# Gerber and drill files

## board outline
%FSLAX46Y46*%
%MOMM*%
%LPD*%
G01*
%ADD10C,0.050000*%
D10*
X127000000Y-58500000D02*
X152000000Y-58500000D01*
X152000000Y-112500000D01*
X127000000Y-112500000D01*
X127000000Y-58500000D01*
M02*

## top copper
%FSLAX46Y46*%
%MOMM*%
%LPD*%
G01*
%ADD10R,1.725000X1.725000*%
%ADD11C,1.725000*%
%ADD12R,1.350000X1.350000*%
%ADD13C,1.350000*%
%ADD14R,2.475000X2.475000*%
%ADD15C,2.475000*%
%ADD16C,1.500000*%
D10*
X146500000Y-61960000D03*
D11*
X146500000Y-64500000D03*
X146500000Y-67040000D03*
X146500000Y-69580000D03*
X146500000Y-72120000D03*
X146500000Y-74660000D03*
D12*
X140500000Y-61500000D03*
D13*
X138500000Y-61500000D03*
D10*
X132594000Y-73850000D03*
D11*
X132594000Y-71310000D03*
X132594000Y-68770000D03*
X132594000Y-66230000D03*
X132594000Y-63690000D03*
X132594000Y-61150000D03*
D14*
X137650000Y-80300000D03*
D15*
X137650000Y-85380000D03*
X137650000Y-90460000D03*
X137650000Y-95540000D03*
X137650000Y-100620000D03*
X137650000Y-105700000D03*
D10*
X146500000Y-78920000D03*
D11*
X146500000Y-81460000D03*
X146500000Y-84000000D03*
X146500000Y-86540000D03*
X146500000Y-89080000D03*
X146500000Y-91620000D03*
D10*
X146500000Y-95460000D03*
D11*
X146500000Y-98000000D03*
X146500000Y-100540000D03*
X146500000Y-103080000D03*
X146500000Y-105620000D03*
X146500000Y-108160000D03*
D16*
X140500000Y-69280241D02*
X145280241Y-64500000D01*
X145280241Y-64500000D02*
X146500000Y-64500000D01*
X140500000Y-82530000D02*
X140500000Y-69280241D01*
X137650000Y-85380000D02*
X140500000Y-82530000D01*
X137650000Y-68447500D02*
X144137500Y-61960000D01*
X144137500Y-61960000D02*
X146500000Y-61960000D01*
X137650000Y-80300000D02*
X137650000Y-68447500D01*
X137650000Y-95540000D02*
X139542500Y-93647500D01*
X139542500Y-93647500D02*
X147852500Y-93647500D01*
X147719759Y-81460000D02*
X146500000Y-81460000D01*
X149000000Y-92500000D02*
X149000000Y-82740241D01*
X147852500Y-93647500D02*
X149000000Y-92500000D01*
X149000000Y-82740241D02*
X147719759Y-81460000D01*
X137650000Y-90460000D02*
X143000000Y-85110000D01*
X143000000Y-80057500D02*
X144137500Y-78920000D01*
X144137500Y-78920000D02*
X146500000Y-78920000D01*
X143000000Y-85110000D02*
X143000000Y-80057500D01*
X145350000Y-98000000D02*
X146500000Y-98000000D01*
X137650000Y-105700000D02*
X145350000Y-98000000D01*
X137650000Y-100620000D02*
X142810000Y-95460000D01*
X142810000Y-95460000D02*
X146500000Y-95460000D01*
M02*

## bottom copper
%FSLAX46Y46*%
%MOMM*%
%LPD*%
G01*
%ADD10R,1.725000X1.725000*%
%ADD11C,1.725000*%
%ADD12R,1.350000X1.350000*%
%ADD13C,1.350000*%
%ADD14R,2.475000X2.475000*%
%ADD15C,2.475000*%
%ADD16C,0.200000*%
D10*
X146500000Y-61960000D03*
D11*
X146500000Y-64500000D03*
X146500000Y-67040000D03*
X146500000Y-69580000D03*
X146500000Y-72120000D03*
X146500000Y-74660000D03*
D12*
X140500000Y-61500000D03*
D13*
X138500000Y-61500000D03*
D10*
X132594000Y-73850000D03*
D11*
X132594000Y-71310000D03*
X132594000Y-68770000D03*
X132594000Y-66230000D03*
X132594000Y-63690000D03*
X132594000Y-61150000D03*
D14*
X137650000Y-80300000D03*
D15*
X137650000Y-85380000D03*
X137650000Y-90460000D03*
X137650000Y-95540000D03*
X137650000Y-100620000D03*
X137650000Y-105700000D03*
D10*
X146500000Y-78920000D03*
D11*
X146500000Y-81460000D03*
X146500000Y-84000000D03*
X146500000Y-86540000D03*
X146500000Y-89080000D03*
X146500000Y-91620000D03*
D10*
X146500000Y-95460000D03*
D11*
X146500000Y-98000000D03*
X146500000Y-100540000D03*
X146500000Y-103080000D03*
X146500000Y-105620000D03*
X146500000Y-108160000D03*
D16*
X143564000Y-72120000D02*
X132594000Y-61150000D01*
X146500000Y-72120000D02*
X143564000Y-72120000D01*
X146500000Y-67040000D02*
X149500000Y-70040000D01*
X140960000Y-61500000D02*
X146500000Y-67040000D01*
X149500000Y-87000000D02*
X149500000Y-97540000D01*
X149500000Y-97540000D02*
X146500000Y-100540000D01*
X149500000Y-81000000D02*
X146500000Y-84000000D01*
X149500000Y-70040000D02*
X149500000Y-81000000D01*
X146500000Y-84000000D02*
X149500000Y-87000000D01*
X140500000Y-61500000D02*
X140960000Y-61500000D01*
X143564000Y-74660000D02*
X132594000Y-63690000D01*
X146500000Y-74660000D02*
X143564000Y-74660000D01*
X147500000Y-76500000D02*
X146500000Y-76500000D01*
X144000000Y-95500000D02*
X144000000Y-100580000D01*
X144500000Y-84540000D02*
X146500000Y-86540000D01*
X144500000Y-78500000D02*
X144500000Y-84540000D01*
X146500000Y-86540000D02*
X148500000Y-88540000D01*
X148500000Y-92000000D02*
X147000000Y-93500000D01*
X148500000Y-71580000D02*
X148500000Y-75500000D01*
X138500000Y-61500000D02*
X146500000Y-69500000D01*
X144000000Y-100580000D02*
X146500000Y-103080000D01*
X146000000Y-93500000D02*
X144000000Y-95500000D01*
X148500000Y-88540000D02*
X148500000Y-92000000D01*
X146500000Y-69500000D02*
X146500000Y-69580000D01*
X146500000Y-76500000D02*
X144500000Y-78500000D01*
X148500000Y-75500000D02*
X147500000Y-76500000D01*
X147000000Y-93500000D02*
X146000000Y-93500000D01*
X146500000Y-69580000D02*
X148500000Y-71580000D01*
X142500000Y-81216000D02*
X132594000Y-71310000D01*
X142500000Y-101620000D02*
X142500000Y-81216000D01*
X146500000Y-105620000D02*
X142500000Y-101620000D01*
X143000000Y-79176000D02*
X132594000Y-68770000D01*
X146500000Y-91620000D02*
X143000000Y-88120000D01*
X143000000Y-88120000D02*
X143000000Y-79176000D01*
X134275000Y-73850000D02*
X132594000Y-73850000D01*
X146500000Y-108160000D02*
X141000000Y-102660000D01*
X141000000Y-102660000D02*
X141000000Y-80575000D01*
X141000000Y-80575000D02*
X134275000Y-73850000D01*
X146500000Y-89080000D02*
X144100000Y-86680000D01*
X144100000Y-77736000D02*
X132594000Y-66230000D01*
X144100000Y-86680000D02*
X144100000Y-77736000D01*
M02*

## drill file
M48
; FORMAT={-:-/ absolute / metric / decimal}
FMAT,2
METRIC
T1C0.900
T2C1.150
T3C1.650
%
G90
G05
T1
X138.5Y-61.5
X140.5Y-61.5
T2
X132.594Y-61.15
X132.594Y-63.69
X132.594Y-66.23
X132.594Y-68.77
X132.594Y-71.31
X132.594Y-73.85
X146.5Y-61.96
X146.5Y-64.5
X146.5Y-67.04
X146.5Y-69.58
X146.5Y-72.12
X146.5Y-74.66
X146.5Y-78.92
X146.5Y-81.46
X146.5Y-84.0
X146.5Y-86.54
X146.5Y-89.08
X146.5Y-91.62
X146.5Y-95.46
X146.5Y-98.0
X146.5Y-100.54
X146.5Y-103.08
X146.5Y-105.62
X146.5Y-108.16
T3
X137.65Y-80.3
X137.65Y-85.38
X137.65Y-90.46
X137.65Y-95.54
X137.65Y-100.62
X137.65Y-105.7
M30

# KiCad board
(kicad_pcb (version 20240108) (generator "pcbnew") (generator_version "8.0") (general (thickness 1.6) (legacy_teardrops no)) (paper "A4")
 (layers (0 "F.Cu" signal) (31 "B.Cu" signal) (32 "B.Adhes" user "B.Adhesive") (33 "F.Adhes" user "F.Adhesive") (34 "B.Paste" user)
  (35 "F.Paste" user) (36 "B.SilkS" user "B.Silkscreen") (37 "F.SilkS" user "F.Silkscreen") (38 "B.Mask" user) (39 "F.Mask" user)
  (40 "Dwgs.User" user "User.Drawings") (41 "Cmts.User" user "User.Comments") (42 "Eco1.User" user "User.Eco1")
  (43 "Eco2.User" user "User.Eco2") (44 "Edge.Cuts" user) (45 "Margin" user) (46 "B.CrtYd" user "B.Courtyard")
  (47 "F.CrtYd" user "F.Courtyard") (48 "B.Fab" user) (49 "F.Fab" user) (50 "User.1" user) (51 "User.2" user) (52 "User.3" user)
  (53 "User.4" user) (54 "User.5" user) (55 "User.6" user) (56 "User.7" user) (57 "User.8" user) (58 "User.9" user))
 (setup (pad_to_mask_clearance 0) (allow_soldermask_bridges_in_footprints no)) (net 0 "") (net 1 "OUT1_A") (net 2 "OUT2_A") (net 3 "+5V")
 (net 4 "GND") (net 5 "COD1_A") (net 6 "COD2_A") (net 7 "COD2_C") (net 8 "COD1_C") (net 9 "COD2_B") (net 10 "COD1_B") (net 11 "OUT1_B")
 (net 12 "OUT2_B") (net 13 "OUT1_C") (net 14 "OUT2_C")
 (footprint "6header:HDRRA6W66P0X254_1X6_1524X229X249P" (layer "F.Cu") (at 146.5 61.96 -90)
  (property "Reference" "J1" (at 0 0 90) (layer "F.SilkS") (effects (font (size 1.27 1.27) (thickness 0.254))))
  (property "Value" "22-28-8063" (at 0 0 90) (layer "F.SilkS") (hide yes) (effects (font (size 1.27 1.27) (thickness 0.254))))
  (pad "1" thru_hole rect (at 0 0 270) (size 1.725 1.725) (drill 1.15) (layers "*.Cu" "*.Mask") (remove_unused_layers no) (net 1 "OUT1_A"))
  (pad "2" thru_hole circle (at 2.54 0 270) (size 1.725 1.725) (drill 1.15) (layers "*.Cu" "*.Mask") (remove_unused_layers no)
   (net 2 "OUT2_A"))
  (pad "3" thru_hole circle (at 5.08 0 270) (size 1.725 1.725) (drill 1.15) (layers "*.Cu" "*.Mask") (remove_unused_layers no) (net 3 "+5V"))
  (pad "4" thru_hole circle (at 7.62 0 270) (size 1.725 1.725) (drill 1.15) (layers "*.Cu" "*.Mask") (remove_unused_layers no) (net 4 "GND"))
  (pad "5" thru_hole circle (at 10.16 0 270) (size 1.725 1.725) (drill 1.15) (layers "*.Cu" "*.Mask") (remove_unused_layers no)
   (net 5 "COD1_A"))
  (pad "6" thru_hole circle (at 12.7 0 270) (size 1.725 1.725) (drill 1.15) (layers "*.Cu" "*.Mask") (remove_unused_layers no)
   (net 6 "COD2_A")))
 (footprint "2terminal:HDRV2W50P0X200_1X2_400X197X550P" (layer "F.Cu") (at 140.5 61.5)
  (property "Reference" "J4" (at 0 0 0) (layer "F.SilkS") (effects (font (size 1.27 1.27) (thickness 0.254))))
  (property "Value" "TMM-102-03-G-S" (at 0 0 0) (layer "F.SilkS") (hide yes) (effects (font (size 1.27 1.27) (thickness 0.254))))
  (pad "1" thru_hole rect (at 0 0) (size 1.35 1.35) (drill 0.9) (layers "*.Cu" "*.Mask") (remove_unused_layers no) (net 3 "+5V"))
  (pad "2" thru_hole circle (at -2 0) (size 1.35 1.35) (drill 0.9) (layers "*.Cu" "*.Mask") (remove_unused_layers no) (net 4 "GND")))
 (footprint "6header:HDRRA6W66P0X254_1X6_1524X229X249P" (layer "F.Cu") (at 132.594 73.85 90)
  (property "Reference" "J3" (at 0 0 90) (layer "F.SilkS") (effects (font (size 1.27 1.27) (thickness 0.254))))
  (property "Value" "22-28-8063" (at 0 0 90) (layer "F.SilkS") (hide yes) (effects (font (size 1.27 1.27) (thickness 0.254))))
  (pad "1" thru_hole rect (at 0 0 90) (size 1.725 1.725) (drill 1.15) (layers "*.Cu" "*.Mask") (remove_unused_layers no) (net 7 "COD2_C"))
  (pad "2" thru_hole circle (at 2.54 0 90) (size 1.725 1.725) (drill 1.15) (layers "*.Cu" "*.Mask") (remove_unused_layers no)
   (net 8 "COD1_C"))
  (pad "3" thru_hole circle (at 5.08 0 90) (size 1.725 1.725) (drill 1.15) (layers "*.Cu" "*.Mask") (remove_unused_layers no)
   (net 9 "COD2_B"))
  (pad "4" thru_hole circle (at 7.62 0 90) (size 1.725 1.725) (drill 1.15) (layers "*.Cu" "*.Mask") (remove_unused_layers no)
   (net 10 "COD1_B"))
  (pad "5" thru_hole circle (at 10.16 0 90) (size 1.725 1.725) (drill 1.15) (layers "*.Cu" "*.Mask") (remove_unused_layers no)
   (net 6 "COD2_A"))
  (pad "6" thru_hole circle (at 12.7 0 90) (size 1.725 1.725) (drill 1.15) (layers "*.Cu" "*.Mask") (remove_unused_layers no)
   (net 5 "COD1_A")))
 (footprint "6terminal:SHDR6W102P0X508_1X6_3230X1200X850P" (layer "F.Cu") (at 137.65 80.3 -90)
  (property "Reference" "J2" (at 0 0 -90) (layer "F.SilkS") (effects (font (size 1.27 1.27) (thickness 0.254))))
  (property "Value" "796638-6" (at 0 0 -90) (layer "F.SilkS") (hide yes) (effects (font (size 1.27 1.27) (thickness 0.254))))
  (pad "1" thru_hole rect (at 0 0 270) (size 2.475 2.475) (drill 1.65) (layers "*.Cu" "*.Mask") (remove_unused_layers no) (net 1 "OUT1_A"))
  (pad "2" thru_hole circle (at 5.08 0 270) (size 2.475 2.475) (drill 1.65) (layers "*.Cu" "*.Mask") (remove_unused_layers no)
   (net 2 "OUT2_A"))
  (pad "3" thru_hole circle (at 10.16 0 270) (size 2.475 2.475) (drill 1.65) (layers "*.Cu" "*.Mask") (remove_unused_layers no)
   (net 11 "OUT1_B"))
  (pad "4" thru_hole circle (at 15.24 0 270) (size 2.475 2.475) (drill 1.65) (layers "*.Cu" "*.Mask") (remove_unused_layers no)
   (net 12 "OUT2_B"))
  (pad "5" thru_hole circle (at 20.32 0 270) (size 2.475 2.475) (drill 1.65) (layers "*.Cu" "*.Mask") (remove_unused_layers no)
   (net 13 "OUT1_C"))
  (pad "6" thru_hole circle (at 25.4 0 270) (size 2.475 2.475) (drill 1.65) (layers "*.Cu" "*.Mask") (remove_unused_layers no)
   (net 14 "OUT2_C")))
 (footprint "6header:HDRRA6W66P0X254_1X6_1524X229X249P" (layer "F.Cu") (at 146.5 78.92 -90)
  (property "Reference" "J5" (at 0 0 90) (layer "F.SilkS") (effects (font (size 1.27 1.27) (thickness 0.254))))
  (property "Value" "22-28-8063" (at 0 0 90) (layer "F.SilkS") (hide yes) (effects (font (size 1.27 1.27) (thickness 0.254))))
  (pad "1" thru_hole rect (at 0 0 270) (size 1.725 1.725) (drill 1.15) (layers "*.Cu" "*.Mask") (remove_unused_layers no) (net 11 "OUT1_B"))
  (pad "2" thru_hole circle (at 2.54 0 270) (size 1.725 1.725) (drill 1.15) (layers "*.Cu" "*.Mask") (remove_unused_layers no)
   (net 12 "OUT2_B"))
  (pad "3" thru_hole circle (at 5.08 0 270) (size 1.725 1.725) (drill 1.15) (layers "*.Cu" "*.Mask") (remove_unused_layers no) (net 3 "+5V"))
  (pad "4" thru_hole circle (at 7.62 0 270) (size 1.725 1.725) (drill 1.15) (layers "*.Cu" "*.Mask") (remove_unused_layers no) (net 4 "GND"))
  (pad "5" thru_hole circle (at 10.16 0 270) (size 1.725 1.725) (drill 1.15) (layers "*.Cu" "*.Mask") (remove_unused_layers no)
   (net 10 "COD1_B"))
  (pad "6" thru_hole circle (at 12.7 0 270) (size 1.725 1.725) (drill 1.15) (layers "*.Cu" "*.Mask") (remove_unused_layers no)
   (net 9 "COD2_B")))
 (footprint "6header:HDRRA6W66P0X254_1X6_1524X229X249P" (layer "F.Cu") (at 146.5 95.46 -90)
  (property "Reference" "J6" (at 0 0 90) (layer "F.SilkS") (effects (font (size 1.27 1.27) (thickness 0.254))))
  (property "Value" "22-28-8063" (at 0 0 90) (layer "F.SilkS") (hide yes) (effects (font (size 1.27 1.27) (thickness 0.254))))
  (pad "1" thru_hole rect (at 0 0 270) (size 1.725 1.725) (drill 1.15) (layers "*.Cu" "*.Mask") (remove_unused_layers no) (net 13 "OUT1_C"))
  (pad "2" thru_hole circle (at 2.54 0 270) (size 1.725 1.725) (drill 1.15) (layers "*.Cu" "*.Mask") (remove_unused_layers no)
   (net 14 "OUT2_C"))
  (pad "3" thru_hole circle (at 5.08 0 270) (size 1.725 1.725) (drill 1.15) (layers "*.Cu" "*.Mask") (remove_unused_layers no) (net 3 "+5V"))
  (pad "4" thru_hole circle (at 7.62 0 270) (size 1.725 1.725) (drill 1.15) (layers "*.Cu" "*.Mask") (remove_unused_layers no) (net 4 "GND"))
  (pad "5" thru_hole circle (at 10.16 0 270) (size 1.725 1.725) (drill 1.15) (layers "*.Cu" "*.Mask") (remove_unused_layers no)
   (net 8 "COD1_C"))
  (pad "6" thru_hole circle (at 12.7 0 270) (size 1.725 1.725) (drill 1.15) (layers "*.Cu" "*.Mask") (remove_unused_layers no)
   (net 7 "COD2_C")))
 (gr_rect (start 127 58.5) (end 152 112.5) (stroke (width 0.05) (type default)) (fill none) (layer "Edge.Cuts"))
 (segment (start 143.564 72.12) (end 132.594 61.15) (width 0.2) (layer "B.Cu") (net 5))
 (segment (start 146.5 72.12) (end 143.564 72.12) (width 0.2) (layer "B.Cu") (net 5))
 (segment (start 140.5 69.280241) (end 145.280241 64.5) (width 1.5) (layer "F.Cu") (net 2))
 (segment (start 145.280241 64.5) (end 146.5 64.5) (width 1.5) (layer "F.Cu") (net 2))
 (segment (start 140.5 82.53) (end 140.5 69.280241) (width 1.5) (layer "F.Cu") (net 2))
 (segment (start 137.65 85.38) (end 140.5 82.53) (width 1.5) (layer "F.Cu") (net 2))
 (segment (start 137.65 68.4475) (end 144.1375 61.96) (width 1.5) (layer "F.Cu") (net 1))
 (segment (start 144.1375 61.96) (end 146.5 61.96) (width 1.5) (layer "F.Cu") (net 1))
 (segment (start 137.65 80.3) (end 137.65 68.4475) (width 1.5) (layer "F.Cu") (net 1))
 (segment (start 146.5 67.04) (end 149.5 70.04) (width 0.2) (layer "B.Cu") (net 3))
 (segment (start 140.96 61.5) (end 146.5 67.04) (width 0.2) (layer "B.Cu") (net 3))
 (segment (start 149.5 87) (end 149.5 97.54) (width 0.2) (layer "B.Cu") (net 3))
 (segment (start 149.5 97.54) (end 146.5 100.54) (width 0.2) (layer "B.Cu") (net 3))
 (segment (start 149.5 81) (end 146.5 84) (width 0.2) (layer "B.Cu") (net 3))
 (segment (start 149.5 70.04) (end 149.5 81) (width 0.2) (layer "B.Cu") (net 3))
 (segment (start 146.5 84) (end 149.5 87) (width 0.2) (layer "B.Cu") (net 3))
 (segment (start 140.5 61.5) (end 140.96 61.5) (width 0.2) (layer "B.Cu") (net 3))
 (segment (start 143.564 74.66) (end 132.594 63.69) (width 0.2) (layer "B.Cu") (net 6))
 (segment (start 146.5 74.66) (end 143.564 74.66) (width 0.2) (layer "B.Cu") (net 6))
 (segment (start 147.5 76.5) (end 146.5 76.5) (width 0.2) (layer "B.Cu") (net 4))
 (segment (start 144 95.5) (end 144 100.58) (width 0.2) (layer "B.Cu") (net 4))
 (segment (start 144.5 84.54) (end 146.5 86.54) (width 0.2) (layer "B.Cu") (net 4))
 (segment (start 144.5 78.5) (end 144.5 84.54) (width 0.2) (layer "B.Cu") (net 4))
 (segment (start 146.5 86.54) (end 148.5 88.54) (width 0.2) (layer "B.Cu") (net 4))
 (segment (start 148.5 92) (end 147 93.5) (width 0.2) (layer "B.Cu") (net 4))
 (segment (start 148.5 71.58) (end 148.5 75.5) (width 0.2) (layer "B.Cu") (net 4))
 (segment (start 138.5 61.5) (end 146.5 69.5) (width 0.2) (layer "B.Cu") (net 4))
 (segment (start 144 100.58) (end 146.5 103.08) (width 0.2) (layer "B.Cu") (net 4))
 (segment (start 146 93.5) (end 144 95.5) (width 0.2) (layer "B.Cu") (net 4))
 (segment (start 148.5 88.54) (end 148.5 92) (width 0.2) (layer "B.Cu") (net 4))
 (segment (start 146.5 69.5) (end 146.5 69.58) (width 0.2) (layer "B.Cu") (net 4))
 (segment (start 146.5 76.5) (end 144.5 78.5) (width 0.2) (layer "B.Cu") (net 4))
 (segment (start 148.5 75.5) (end 147.5 76.5) (width 0.2) (layer "B.Cu") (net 4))
 (segment (start 147 93.5) (end 146 93.5) (width 0.2) (layer "B.Cu") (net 4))
 (segment (start 146.5 69.58) (end 148.5 71.58) (width 0.2) (layer "B.Cu") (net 4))
 (segment (start 142.5 81.216) (end 132.594 71.31) (width 0.2) (layer "B.Cu") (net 8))
 (segment (start 142.5 101.62) (end 142.5 81.216) (width 0.2) (layer "B.Cu") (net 8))
 (segment (start 146.5 105.62) (end 142.5 101.62) (width 0.2) (layer "B.Cu") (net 8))
 (segment (start 143 79.176) (end 132.594 68.77) (width 0.2) (layer "B.Cu") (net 9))
 (segment (start 146.5 91.62) (end 143 88.12) (width 0.2) (layer "B.Cu") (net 9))
 (segment (start 143 88.12) (end 143 79.176) (width 0.2) (layer "B.Cu") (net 9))
 (segment (start 134.275 73.85) (end 132.594 73.85) (width 0.2) (layer "B.Cu") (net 7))
 (segment (start 146.5 108.16) (end 141 102.66) (width 0.2) (layer "B.Cu") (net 7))
 (segment (start 141 102.66) (end 141 80.575) (width 0.2) (layer "B.Cu") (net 7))
 (segment (start 141 80.575) (end 134.275 73.85) (width 0.2) (layer "B.Cu") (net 7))
 (segment (start 146.5 89.08) (end 144.1 86.68) (width 0.2) (layer "B.Cu") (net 10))
 (segment (start 144.1 77.736) (end 132.594 66.23) (width 0.2) (layer "B.Cu") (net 10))
 (segment (start 144.1 86.68) (end 144.1 77.736) (width 0.2) (layer "B.Cu") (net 10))
 (segment (start 137.65 95.54) (end 139.5425 93.6475) (width 1.5) (layer "F.Cu") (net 12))
 (segment (start 139.5425 93.6475) (end 147.8525 93.6475) (width 1.5) (layer "F.Cu") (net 12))
 (segment (start 147.719759 81.46) (end 146.5 81.46) (width 1.5) (layer "F.Cu") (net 12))
 (segment (start 149 92.5) (end 149 82.740241) (width 1.5) (layer "F.Cu") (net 12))
 (segment (start 147.8525 93.6475) (end 149 92.5) (width 1.5) (layer "F.Cu") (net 12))
 (segment (start 149 82.740241) (end 147.719759 81.46) (width 1.5) (layer "F.Cu") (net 12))
 (segment (start 137.65 90.46) (end 143 85.11) (width 1.5) (layer "F.Cu") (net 11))
 (segment (start 143 80.0575) (end 144.1375 78.92) (width 1.5) (layer "F.Cu") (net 11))
 (segment (start 144.1375 78.92) (end 146.5 78.92) (width 1.5) (layer "F.Cu") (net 11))
 (segment (start 143 85.11) (end 143 80.0575) (width 1.5) (layer "F.Cu") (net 11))
 (segment (start 145.35 98) (end 146.5 98) (width 1.5) (layer "F.Cu") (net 14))
 (segment (start 137.65 105.7) (end 145.35 98) (width 1.5) (layer "F.Cu") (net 14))
 (segment (start 137.65 100.62) (end 142.81 95.46) (width 1.5) (layer "F.Cu") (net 13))
 (segment (start 142.81 95.46) (end 146.5 95.46) (width 1.5) (layer "F.Cu") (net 13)))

